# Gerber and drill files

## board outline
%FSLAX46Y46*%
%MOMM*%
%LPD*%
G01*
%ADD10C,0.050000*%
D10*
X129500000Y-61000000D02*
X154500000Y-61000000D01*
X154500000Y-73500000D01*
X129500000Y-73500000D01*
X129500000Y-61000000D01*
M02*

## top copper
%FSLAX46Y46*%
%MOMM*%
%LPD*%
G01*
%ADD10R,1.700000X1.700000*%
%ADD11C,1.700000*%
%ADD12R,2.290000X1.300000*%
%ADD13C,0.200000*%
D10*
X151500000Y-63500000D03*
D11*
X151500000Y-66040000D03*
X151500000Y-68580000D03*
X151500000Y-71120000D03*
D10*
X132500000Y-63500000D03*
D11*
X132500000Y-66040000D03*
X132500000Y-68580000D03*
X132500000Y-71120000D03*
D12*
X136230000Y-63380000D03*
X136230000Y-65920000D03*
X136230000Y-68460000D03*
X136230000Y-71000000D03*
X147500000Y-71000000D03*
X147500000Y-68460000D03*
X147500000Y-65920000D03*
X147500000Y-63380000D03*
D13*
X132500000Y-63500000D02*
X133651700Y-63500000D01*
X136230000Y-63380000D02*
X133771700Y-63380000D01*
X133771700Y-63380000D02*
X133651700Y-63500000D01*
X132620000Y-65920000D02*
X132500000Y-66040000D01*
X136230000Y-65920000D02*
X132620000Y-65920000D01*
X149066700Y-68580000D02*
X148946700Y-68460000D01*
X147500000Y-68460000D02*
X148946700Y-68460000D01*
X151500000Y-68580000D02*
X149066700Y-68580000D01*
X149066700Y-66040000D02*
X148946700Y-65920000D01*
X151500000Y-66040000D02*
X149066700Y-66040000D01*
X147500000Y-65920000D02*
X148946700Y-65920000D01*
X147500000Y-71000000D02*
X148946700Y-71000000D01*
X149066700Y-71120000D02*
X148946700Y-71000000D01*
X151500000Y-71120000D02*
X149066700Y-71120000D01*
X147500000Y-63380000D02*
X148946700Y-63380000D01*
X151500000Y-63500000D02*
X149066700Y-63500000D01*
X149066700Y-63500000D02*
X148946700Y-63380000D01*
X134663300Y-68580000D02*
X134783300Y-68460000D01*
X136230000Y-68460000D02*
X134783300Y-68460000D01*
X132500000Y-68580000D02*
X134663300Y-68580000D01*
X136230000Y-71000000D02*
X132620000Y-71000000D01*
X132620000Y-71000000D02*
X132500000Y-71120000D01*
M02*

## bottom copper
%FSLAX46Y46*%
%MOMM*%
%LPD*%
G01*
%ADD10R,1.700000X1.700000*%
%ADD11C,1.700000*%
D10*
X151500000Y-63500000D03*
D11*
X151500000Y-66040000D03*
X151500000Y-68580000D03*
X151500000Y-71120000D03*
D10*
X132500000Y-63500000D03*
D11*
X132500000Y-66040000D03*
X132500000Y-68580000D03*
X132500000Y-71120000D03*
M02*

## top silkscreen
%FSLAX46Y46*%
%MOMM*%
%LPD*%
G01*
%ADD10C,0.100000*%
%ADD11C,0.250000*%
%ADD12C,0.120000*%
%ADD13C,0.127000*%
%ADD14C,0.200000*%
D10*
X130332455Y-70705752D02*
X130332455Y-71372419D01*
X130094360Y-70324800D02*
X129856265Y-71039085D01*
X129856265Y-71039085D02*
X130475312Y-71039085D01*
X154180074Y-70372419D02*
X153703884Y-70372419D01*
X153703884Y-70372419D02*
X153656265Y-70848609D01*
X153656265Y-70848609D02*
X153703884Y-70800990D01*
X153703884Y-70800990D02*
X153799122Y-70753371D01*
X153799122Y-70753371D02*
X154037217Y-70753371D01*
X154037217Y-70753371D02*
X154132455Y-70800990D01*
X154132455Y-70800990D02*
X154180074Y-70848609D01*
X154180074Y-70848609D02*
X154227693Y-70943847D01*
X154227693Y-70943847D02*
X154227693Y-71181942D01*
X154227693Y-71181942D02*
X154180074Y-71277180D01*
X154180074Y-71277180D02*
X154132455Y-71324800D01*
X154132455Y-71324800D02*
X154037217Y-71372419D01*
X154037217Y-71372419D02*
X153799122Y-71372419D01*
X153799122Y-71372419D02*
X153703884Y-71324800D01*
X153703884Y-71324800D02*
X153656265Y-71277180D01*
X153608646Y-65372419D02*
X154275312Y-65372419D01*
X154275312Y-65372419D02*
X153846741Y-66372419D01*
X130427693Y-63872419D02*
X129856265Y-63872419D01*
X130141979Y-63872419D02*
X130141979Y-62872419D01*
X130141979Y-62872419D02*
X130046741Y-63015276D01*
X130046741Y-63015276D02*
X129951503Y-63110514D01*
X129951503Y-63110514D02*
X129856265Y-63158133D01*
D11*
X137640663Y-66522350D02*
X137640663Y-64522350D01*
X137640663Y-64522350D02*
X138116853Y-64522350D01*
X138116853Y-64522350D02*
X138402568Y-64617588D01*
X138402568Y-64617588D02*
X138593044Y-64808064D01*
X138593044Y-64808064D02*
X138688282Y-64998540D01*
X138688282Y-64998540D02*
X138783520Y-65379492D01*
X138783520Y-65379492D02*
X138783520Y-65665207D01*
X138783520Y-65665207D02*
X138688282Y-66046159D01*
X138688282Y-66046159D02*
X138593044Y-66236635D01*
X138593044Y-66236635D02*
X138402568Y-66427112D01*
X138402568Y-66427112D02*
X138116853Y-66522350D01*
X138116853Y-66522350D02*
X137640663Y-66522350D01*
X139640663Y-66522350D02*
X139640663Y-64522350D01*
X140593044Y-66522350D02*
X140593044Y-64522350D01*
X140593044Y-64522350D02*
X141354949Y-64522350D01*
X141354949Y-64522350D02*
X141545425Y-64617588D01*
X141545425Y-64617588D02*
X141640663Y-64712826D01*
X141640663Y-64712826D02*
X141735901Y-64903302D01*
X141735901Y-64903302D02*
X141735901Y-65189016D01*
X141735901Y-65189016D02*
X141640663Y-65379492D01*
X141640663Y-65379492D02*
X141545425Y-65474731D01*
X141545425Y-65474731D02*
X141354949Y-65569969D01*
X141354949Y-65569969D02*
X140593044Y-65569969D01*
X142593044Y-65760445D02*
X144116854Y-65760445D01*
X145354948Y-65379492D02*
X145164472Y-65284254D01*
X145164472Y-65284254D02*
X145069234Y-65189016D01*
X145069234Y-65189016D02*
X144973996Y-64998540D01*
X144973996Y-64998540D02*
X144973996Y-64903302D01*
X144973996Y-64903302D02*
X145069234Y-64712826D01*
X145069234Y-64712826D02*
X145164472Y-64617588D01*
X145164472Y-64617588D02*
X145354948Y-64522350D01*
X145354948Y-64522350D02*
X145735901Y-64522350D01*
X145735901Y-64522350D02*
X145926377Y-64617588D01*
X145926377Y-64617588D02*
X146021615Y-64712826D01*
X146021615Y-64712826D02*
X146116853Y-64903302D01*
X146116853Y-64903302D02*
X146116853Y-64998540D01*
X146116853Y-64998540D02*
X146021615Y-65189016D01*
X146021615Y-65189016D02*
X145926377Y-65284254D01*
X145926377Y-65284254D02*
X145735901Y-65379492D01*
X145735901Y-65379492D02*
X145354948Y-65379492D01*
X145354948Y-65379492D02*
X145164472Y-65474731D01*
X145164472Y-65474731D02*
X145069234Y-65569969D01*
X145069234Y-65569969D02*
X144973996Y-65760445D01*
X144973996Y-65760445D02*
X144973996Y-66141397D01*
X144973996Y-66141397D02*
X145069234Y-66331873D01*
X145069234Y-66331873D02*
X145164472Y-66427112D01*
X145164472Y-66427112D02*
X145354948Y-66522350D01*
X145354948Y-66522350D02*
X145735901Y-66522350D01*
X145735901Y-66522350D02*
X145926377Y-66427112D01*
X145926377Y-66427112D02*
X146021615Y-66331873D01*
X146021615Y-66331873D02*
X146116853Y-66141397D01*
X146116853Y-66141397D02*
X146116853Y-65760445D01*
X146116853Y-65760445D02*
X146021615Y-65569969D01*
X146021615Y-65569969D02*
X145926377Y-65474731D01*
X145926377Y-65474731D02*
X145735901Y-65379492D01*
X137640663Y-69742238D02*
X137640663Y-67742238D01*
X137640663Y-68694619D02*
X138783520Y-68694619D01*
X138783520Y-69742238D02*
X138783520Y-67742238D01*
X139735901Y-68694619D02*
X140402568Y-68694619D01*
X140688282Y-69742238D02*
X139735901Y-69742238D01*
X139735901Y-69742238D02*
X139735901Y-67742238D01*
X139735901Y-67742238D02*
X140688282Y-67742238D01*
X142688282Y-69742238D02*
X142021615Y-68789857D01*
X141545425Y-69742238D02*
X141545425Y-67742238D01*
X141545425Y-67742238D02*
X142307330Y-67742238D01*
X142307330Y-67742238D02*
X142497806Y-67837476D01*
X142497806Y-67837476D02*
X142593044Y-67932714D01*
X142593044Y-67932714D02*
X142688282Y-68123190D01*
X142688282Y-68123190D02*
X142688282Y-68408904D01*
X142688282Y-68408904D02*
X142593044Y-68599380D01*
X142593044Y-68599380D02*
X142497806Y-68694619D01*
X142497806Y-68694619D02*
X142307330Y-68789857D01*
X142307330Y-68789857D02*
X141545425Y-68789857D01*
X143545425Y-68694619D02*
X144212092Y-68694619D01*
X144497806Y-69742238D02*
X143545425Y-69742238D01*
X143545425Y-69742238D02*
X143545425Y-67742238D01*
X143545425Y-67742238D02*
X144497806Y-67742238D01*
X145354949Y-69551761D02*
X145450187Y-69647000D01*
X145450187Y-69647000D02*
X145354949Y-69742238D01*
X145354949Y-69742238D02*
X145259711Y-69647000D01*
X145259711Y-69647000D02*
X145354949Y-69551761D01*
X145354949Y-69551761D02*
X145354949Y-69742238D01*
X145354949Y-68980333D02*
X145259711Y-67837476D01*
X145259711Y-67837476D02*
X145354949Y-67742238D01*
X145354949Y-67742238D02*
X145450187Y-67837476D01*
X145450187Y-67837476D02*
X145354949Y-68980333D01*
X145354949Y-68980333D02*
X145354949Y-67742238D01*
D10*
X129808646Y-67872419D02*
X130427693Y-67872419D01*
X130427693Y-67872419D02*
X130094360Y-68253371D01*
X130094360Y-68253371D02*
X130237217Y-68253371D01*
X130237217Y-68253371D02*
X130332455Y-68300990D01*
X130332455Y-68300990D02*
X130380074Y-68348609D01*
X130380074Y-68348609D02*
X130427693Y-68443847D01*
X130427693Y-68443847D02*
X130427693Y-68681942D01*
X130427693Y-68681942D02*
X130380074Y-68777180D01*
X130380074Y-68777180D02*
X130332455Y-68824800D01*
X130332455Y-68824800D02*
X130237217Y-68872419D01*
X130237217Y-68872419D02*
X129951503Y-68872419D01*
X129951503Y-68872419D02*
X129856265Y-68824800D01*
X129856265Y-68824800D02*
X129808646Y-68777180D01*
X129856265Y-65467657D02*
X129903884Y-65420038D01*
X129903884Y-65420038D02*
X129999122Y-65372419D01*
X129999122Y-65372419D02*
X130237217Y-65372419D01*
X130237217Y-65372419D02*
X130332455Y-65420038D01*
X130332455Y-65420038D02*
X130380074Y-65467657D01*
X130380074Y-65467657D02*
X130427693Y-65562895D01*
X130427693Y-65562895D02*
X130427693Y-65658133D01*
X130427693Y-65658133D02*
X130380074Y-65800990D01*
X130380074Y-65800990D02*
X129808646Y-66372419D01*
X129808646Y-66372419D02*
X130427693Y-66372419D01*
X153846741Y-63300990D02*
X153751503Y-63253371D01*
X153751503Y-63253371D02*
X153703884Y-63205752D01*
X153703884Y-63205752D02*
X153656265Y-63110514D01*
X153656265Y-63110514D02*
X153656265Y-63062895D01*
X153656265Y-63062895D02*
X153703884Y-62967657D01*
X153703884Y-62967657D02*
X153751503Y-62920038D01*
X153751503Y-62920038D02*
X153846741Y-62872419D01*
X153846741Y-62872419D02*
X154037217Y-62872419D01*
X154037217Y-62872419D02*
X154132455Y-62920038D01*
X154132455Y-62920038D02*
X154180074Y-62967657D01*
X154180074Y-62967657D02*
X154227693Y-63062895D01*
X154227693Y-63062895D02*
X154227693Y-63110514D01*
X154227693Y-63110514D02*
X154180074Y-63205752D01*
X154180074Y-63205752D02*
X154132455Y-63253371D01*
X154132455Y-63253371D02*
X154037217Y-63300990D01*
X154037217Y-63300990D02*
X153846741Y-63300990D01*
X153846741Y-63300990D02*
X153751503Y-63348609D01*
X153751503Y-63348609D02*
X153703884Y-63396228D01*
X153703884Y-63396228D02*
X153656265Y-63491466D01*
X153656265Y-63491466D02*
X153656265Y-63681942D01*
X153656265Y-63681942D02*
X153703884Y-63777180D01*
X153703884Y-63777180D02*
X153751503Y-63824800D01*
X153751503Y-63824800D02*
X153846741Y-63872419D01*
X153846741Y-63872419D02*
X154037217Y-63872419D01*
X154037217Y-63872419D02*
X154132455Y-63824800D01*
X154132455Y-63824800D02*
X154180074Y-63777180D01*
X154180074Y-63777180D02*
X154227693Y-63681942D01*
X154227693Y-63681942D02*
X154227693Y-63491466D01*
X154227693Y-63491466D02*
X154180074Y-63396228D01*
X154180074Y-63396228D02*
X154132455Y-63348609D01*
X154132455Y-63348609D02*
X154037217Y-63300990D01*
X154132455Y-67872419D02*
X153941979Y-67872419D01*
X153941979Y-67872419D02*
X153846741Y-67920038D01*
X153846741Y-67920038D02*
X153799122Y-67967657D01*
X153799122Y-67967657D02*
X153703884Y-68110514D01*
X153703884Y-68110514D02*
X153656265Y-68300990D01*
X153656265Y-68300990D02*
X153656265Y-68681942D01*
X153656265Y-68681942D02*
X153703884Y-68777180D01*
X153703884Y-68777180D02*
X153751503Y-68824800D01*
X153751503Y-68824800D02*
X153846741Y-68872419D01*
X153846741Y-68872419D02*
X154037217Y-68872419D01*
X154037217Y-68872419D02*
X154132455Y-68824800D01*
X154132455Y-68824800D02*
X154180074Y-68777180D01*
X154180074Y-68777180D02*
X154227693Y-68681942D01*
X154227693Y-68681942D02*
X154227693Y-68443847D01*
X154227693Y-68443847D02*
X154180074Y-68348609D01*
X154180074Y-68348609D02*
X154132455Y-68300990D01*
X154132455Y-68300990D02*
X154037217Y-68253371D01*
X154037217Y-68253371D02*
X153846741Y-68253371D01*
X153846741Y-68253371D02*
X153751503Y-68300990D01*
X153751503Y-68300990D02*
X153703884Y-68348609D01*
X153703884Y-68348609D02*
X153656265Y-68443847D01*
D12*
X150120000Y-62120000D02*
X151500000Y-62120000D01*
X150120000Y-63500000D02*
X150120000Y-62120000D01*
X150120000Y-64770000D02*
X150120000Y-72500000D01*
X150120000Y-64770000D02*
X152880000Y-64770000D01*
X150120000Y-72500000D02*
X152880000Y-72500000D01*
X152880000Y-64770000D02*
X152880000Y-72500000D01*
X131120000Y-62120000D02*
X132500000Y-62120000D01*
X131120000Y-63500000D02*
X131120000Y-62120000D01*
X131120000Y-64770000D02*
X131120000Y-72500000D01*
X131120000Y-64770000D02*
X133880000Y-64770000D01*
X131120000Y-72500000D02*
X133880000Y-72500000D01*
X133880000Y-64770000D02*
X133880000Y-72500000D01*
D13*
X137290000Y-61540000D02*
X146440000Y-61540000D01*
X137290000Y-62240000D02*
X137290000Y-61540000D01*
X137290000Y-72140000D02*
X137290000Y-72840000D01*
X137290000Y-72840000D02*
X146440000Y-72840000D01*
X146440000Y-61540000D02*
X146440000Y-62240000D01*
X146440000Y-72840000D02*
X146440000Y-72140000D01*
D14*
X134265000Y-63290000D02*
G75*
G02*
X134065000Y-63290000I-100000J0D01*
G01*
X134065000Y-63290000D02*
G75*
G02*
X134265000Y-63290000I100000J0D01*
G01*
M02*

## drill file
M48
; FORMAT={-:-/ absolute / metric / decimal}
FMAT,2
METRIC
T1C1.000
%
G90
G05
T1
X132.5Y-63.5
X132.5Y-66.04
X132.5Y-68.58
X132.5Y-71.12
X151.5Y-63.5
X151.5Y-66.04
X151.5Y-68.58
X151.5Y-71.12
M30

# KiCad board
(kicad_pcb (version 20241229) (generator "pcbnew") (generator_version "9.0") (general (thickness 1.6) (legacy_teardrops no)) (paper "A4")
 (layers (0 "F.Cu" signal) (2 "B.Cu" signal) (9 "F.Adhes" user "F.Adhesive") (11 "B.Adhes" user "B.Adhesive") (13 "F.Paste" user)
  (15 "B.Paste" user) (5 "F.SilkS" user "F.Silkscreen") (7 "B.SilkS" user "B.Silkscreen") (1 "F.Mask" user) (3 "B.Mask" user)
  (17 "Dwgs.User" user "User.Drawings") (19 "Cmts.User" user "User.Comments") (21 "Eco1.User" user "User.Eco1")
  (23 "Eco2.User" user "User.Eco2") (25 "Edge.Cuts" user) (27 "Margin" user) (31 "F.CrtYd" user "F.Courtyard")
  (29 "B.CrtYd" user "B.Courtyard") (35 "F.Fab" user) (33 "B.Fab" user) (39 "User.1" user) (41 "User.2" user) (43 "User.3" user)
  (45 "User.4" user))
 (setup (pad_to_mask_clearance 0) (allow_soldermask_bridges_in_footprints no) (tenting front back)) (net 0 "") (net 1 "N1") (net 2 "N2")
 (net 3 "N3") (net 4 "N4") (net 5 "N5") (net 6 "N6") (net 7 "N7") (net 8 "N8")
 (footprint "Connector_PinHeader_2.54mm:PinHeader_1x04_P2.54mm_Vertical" (layer "F.Cu") (at 151.5 63.5)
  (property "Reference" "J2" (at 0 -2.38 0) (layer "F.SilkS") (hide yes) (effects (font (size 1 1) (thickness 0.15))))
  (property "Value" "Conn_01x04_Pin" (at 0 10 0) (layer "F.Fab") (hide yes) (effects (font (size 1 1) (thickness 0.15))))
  (fp_line (start -1.38 -1.38) (end 0 -1.38) (stroke (width 0.12) (type solid)) (layer "F.SilkS"))
  (fp_line (start -1.38 0) (end -1.38 -1.38) (stroke (width 0.12) (type solid)) (layer "F.SilkS"))
  (fp_line (start -1.38 1.27) (end -1.38 9) (stroke (width 0.12) (type solid)) (layer "F.SilkS"))
  (fp_line (start -1.38 1.27) (end 1.38 1.27) (stroke (width 0.12) (type solid)) (layer "F.SilkS"))
  (fp_line (start -1.38 9) (end 1.38 9) (stroke (width 0.12) (type solid)) (layer "F.SilkS"))
  (fp_line (start 1.38 1.27) (end 1.38 9) (stroke (width 0.12) (type solid)) (layer "F.SilkS"))
  (pad "1" thru_hole rect (at 0 0) (size 1.7 1.7) (drill 1) (layers "*.Cu" "*.Mask") (remove_unused_layers no) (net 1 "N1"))
  (pad "2" thru_hole circle (at 0 2.54) (size 1.7 1.7) (drill 1) (layers "*.Cu" "*.Mask") (remove_unused_layers no) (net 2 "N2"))
  (pad "3" thru_hole circle (at 0 5.08) (size 1.7 1.7) (drill 1) (layers "*.Cu" "*.Mask") (remove_unused_layers no) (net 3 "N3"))
  (pad "4" thru_hole circle (at 0 7.62) (size 1.7 1.7) (drill 1) (layers "*.Cu" "*.Mask") (remove_unused_layers no) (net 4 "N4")))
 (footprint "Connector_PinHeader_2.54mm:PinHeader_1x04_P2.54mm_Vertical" (layer "F.Cu") (at 132.5 63.5)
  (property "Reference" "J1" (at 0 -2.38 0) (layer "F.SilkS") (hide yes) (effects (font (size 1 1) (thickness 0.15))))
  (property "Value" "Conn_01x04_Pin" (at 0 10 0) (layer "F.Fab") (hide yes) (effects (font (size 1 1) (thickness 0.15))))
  (fp_line (start -1.38 -1.38) (end 0 -1.38) (stroke (width 0.12) (type solid)) (layer "F.SilkS"))
  (fp_line (start -1.38 0) (end -1.38 -1.38) (stroke (width 0.12) (type solid)) (layer "F.SilkS"))
  (fp_line (start -1.38 1.27) (end -1.38 9) (stroke (width 0.12) (type solid)) (layer "F.SilkS"))
  (fp_line (start -1.38 1.27) (end 1.38 1.27) (stroke (width 0.12) (type solid)) (layer "F.SilkS"))
  (fp_line (start -1.38 9) (end 1.38 9) (stroke (width 0.12) (type solid)) (layer "F.SilkS"))
  (fp_line (start 1.38 1.27) (end 1.38 9) (stroke (width 0.12) (type solid)) (layer "F.SilkS"))
  (pad "1" thru_hole rect (at 0 0) (size 1.7 1.7) (drill 1) (layers "*.Cu" "*.Mask") (remove_unused_layers no) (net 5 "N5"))
  (pad "2" thru_hole circle (at 0 2.54) (size 1.7 1.7) (drill 1) (layers "*.Cu" "*.Mask") (remove_unused_layers no) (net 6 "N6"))
  (pad "3" thru_hole circle (at 0 5.08) (size 1.7 1.7) (drill 1) (layers "*.Cu" "*.Mask") (remove_unused_layers no) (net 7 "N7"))
  (pad "4" thru_hole circle (at 0 7.62) (size 1.7 1.7) (drill 1) (layers "*.Cu" "*.Mask") (remove_unused_layers no) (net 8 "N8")))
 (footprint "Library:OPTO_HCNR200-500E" (layer "F.Cu") (at 141.865 67.19)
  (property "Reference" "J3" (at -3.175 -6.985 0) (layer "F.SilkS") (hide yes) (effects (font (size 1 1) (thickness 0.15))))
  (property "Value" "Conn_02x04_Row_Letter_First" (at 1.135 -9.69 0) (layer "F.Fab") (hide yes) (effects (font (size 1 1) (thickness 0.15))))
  (fp_line (start -4.575 -5.65) (end 4.575 -5.65) (stroke (width 0.127) (type solid)) (layer "F.SilkS"))
  (fp_line (start -4.575 -4.95) (end -4.575 -5.65) (stroke (width 0.127) (type solid)) (layer "F.SilkS"))
  (fp_line (start -4.575 4.95) (end -4.575 5.65) (stroke (width 0.127) (type solid)) (layer "F.SilkS"))
  (fp_line (start -4.575 5.65) (end 4.575 5.65) (stroke (width 0.127) (type solid)) (layer "F.SilkS"))
  (fp_line (start 4.575 -5.65) (end 4.575 -4.95) (stroke (width 0.127) (type solid)) (layer "F.SilkS"))
  (fp_line (start 4.575 5.65) (end 4.575 4.95) (stroke (width 0.127) (type solid)) (layer "F.SilkS"))
  (fp_circle (center -7.7 -3.9) (end -7.6 -3.9) (stroke (width 0.2) (type solid)) (fill no) (layer "F.SilkS"))
  (pad "1" smd rect (at -5.635 -3.81) (size 2.29 1.3) (layers "F.Cu" "F.Mask" "F.Paste") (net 5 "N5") (solder_mask_margin 0.102))
  (pad "2" smd rect (at -5.635 -1.27) (size 2.29 1.3) (layers "F.Cu" "F.Mask" "F.Paste") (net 6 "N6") (solder_mask_margin 0.102))
  (pad "3" smd rect (at -5.635 1.27) (size 2.29 1.3) (layers "F.Cu" "F.Mask" "F.Paste") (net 7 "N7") (solder_mask_margin 0.102))
  (pad "4" smd rect (at -5.635 3.81) (size 2.29 1.3) (layers "F.Cu" "F.Mask" "F.Paste") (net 8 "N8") (solder_mask_margin 0.102))
  (pad "5" smd rect (at 5.635 3.81) (size 2.29 1.3) (layers "F.Cu" "F.Mask" "F.Paste") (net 4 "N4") (solder_mask_margin 0.102))
  (pad "6" smd rect (at 5.635 1.27) (size 2.29 1.3) (layers "F.Cu" "F.Mask" "F.Paste") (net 3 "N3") (solder_mask_margin 0.102))
  (pad "7" smd rect (at 5.635 -1.27) (size 2.29 1.3) (layers "F.Cu" "F.Mask" "F.Paste") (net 2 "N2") (solder_mask_margin 0.102))
  (pad "8" smd rect (at 5.635 -3.81) (size 2.29 1.3) (layers "F.Cu" "F.Mask" "F.Paste") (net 1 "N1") (solder_mask_margin 0.102)))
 (gr_rect (start 129.5 61) (end 154.5 73.5) (stroke (width 0.05) (type default)) (fill no) (layer "Edge.Cuts"))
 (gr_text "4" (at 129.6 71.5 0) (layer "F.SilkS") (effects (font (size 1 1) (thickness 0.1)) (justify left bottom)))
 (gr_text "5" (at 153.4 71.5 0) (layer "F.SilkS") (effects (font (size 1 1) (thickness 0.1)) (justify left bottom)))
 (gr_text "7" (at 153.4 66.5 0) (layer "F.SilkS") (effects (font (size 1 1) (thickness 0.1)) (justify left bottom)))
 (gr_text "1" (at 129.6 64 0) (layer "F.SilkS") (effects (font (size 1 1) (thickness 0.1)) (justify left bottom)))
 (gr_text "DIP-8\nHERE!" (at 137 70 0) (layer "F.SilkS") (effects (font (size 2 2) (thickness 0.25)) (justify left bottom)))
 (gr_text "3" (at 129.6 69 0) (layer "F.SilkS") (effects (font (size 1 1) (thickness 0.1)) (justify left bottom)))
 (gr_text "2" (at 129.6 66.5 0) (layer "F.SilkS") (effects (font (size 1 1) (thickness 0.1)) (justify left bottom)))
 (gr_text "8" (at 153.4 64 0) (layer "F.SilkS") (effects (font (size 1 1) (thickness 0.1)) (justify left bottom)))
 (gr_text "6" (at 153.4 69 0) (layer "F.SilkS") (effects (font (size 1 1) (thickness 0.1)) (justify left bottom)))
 (segment (start 132.5 63.5) (end 133.6517 63.5) (width 0.2) (layer "F.Cu") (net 5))
 (segment (start 136.23 63.38) (end 133.7717 63.38) (width 0.2) (layer "F.Cu") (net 5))
 (segment (start 133.7717 63.38) (end 133.6517 63.5) (width 0.2) (layer "F.Cu") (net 5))
 (segment (start 132.62 65.92) (end 132.5 66.04) (width 0.2) (layer "F.Cu") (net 6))
 (segment (start 136.23 65.92) (end 132.62 65.92) (width 0.2) (layer "F.Cu") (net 6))
 (segment (start 149.0667 68.58) (end 148.9467 68.46) (width 0.2) (layer "F.Cu") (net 3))
 (segment (start 147.5 68.46) (end 148.9467 68.46) (width 0.2) (layer "F.Cu") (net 3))
 (segment (start 151.5 68.58) (end 149.0667 68.58) (width 0.2) (layer "F.Cu") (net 3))
 (segment (start 149.0667 66.04) (end 148.9467 65.92) (width 0.2) (layer "F.Cu") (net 2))
 (segment (start 151.5 66.04) (end 149.0667 66.04) (width 0.2) (layer "F.Cu") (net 2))
 (segment (start 147.5 65.92) (end 148.9467 65.92) (width 0.2) (layer "F.Cu") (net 2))
 (segment (start 147.5 71) (end 148.9467 71) (width 0.2) (layer "F.Cu") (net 4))
 (segment (start 149.0667 71.12) (end 148.9467 71) (width 0.2) (layer "F.Cu") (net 4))
 (segment (start 151.5 71.12) (end 149.0667 71.12) (width 0.2) (layer "F.Cu") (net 4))
 (segment (start 147.5 63.38) (end 148.9467 63.38) (width 0.2) (layer "F.Cu") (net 1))
 (segment (start 151.5 63.5) (end 149.0667 63.5) (width 0.2) (layer "F.Cu") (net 1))
 (segment (start 149.0667 63.5) (end 148.9467 63.38) (width 0.2) (layer "F.Cu") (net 1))
 (segment (start 134.6633 68.58) (end 134.7833 68.46) (width 0.2) (layer "F.Cu") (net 7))
 (segment (start 136.23 68.46) (end 134.7833 68.46) (width 0.2) (layer "F.Cu") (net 7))
 (segment (start 132.5 68.58) (end 134.6633 68.58) (width 0.2) (layer "F.Cu") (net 7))
 (segment (start 136.23 71) (end 132.62 71) (width 0.2) (layer "F.Cu") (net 8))
 (segment (start 132.62 71) (end 132.5 71.12) (width 0.2) (layer "F.Cu") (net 8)))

